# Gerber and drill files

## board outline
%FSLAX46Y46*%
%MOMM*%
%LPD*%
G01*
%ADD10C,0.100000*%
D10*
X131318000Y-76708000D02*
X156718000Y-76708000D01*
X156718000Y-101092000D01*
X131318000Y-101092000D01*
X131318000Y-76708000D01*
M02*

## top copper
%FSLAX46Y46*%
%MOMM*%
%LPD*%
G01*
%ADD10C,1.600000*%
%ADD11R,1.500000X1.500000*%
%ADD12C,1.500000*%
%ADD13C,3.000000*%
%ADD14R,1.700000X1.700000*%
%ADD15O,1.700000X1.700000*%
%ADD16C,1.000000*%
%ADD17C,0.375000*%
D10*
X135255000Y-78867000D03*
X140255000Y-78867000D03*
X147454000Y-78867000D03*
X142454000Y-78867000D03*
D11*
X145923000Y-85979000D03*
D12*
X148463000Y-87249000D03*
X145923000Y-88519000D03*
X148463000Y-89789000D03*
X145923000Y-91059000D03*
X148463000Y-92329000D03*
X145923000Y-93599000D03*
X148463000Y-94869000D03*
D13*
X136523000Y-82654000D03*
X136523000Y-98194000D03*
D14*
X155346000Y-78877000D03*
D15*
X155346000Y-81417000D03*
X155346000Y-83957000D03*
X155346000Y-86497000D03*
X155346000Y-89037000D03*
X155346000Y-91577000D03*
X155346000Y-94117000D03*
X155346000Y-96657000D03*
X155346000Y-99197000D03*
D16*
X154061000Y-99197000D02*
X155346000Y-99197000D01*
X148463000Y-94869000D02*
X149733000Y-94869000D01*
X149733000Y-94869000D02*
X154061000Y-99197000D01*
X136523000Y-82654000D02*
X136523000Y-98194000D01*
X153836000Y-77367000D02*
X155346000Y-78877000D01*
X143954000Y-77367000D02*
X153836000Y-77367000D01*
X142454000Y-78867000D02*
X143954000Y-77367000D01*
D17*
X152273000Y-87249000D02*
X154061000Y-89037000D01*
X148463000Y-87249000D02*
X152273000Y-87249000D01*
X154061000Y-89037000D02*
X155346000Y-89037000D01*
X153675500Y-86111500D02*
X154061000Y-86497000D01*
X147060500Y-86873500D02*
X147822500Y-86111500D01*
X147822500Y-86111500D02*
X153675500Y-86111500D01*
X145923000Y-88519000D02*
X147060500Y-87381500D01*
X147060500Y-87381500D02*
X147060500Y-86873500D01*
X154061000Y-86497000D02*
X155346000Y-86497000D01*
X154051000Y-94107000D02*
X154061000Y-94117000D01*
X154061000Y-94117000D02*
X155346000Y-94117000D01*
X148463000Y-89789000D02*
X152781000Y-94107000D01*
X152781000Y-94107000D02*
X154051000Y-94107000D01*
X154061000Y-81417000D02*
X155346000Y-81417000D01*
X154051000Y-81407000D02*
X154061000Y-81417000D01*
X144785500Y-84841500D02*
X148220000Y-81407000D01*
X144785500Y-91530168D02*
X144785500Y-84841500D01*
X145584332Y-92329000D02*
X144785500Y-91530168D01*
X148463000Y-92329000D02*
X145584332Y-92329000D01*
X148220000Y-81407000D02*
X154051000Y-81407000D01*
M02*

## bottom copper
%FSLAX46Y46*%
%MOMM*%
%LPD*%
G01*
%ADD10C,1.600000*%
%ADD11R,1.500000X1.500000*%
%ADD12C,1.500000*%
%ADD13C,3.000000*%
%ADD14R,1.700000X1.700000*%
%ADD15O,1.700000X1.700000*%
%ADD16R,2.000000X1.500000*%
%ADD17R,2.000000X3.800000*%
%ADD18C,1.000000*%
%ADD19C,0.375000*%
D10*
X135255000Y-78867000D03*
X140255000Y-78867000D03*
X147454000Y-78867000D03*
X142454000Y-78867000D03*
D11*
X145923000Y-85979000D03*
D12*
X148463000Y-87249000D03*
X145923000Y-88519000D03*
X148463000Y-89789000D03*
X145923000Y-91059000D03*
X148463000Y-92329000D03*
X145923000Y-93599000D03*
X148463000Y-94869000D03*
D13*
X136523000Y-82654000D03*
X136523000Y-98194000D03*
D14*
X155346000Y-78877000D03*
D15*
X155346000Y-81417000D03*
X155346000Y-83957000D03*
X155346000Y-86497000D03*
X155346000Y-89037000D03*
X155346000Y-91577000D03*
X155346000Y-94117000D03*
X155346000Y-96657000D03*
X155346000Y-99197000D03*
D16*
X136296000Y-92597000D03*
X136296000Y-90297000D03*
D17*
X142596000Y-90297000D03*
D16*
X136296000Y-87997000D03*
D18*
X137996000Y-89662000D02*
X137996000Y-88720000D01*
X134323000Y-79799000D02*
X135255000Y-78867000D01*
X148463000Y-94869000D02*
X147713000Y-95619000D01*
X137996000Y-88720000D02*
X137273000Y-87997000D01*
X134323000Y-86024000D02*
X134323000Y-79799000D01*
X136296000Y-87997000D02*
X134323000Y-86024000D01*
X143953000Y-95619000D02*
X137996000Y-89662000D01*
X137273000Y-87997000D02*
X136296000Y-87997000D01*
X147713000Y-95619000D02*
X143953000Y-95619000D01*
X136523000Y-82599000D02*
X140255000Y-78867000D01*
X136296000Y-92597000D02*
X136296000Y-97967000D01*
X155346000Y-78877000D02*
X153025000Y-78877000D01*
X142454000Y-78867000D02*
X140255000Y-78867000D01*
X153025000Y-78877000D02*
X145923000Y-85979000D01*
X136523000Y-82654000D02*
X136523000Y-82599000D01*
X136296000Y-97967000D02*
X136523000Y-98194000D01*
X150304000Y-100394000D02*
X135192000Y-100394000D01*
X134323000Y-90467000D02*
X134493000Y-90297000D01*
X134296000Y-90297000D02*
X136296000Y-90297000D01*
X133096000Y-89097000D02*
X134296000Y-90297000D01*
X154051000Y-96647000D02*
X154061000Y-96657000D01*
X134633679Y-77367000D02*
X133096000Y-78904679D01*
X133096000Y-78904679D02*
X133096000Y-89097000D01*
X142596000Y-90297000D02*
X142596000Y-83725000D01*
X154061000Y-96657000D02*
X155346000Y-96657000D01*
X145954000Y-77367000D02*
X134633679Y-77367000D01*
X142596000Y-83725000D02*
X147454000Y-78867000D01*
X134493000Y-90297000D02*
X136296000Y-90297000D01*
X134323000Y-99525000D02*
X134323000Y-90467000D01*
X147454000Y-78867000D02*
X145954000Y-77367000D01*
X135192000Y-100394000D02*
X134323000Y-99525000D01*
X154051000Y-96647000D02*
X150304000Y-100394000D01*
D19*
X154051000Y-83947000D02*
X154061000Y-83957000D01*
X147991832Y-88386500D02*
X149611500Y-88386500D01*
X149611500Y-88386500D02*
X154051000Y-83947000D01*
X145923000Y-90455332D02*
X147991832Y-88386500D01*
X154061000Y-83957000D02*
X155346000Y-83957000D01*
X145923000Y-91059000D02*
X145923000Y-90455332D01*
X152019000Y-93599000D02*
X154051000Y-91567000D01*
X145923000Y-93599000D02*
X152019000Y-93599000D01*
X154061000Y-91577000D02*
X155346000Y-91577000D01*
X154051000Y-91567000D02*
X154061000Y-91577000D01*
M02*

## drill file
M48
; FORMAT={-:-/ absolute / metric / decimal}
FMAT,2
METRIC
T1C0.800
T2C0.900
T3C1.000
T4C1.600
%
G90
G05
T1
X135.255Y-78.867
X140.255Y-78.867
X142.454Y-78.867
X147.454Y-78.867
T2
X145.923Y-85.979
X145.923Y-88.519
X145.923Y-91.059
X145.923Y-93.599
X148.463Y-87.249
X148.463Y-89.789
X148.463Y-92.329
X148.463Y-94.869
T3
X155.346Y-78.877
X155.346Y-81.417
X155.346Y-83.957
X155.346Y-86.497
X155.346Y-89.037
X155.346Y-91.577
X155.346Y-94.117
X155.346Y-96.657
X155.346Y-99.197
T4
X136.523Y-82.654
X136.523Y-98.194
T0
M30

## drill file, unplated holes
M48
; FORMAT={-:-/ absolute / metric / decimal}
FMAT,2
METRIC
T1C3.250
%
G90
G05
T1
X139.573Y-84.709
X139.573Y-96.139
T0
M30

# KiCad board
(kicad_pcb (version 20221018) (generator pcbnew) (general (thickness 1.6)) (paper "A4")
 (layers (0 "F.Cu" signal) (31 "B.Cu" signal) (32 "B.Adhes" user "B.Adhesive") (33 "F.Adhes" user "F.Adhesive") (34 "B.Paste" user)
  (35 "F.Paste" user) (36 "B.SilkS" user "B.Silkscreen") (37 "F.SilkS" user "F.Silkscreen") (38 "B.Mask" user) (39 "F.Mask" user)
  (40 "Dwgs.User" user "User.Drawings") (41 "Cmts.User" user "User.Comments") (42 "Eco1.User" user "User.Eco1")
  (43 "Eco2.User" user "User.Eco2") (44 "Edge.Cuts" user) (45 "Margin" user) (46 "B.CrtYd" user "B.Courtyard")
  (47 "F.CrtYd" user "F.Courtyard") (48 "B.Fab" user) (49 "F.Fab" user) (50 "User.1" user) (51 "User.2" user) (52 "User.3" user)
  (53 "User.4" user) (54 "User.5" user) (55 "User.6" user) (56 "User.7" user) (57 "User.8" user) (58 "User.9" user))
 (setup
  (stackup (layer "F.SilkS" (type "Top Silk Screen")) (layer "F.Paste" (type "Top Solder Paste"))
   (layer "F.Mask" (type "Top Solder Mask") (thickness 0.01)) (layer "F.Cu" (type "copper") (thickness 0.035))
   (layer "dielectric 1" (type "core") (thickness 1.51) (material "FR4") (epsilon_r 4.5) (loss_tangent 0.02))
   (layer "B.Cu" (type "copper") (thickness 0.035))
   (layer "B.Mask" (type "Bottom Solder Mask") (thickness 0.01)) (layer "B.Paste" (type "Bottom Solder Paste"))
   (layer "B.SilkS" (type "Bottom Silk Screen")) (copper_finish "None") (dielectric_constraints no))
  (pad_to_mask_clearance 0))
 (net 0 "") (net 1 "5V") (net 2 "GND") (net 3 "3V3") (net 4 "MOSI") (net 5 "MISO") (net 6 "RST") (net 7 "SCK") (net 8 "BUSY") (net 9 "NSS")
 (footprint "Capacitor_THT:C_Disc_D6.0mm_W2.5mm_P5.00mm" (layer "F.Cu") (at 135.255 78.867)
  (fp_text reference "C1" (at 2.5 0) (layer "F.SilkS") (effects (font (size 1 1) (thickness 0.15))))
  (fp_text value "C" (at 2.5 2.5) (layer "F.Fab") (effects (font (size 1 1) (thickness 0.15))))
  (pad "1" thru_hole circle (at 0 0) (size 1.6 1.6) (drill 0.8) (layers "*.Cu" "*.Mask") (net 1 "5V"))
  (pad "2" thru_hole circle (at 5 0) (size 1.6 1.6) (drill 0.8) (layers "*.Cu" "*.Mask") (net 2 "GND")))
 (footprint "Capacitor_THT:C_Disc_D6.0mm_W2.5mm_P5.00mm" (layer "F.Cu") (at 147.454 78.867 180)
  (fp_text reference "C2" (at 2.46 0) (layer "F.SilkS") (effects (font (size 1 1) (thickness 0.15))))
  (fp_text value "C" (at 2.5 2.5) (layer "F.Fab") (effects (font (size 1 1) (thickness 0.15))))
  (pad "1" thru_hole circle (at 0 0 180) (size 1.6 1.6) (drill 0.8) (layers "*.Cu" "*.Mask") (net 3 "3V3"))
  (pad "2" thru_hole circle (at 5 0 180) (size 1.6 1.6) (drill 0.8) (layers "*.Cu" "*.Mask") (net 2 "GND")))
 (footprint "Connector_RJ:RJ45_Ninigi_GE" (layer "F.Cu") (at 145.923 85.979 -90)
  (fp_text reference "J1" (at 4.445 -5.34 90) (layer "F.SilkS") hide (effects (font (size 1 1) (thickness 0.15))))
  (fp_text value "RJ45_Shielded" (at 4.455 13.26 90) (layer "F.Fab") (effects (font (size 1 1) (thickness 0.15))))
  (pad "" np_thru_hole circle (at -1.27 6.35 270) (size 3.25 3.25) (drill 3.25) (layers "*.Cu" "*.Mask"))
  (pad "" np_thru_hole circle (at 10.16 6.35 90) (size 3.25 3.25) (drill 3.25) (layers "*.Cu" "*.Mask"))
  (pad "1" thru_hole rect (at 0 0 90) (size 1.5 1.5) (drill 0.9) (layers "*.Cu" "*.Mask") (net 2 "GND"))
  (pad "2" thru_hole circle (at 1.27 -2.54 90) (size 1.5 1.5) (drill 0.9) (layers "*.Cu" "*.Mask") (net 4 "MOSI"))
  (pad "3" thru_hole circle (at 2.54 0 90) (size 1.5 1.5) (drill 0.9) (layers "*.Cu" "*.Mask") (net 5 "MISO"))
  (pad "4" thru_hole circle (at 3.81 -2.54 90) (size 1.5 1.5) (drill 0.9) (layers "*.Cu" "*.Mask") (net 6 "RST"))
  (pad "5" thru_hole circle (at 5.08 0 90) (size 1.5 1.5) (drill 0.9) (layers "*.Cu" "*.Mask") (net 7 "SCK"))
  (pad "6" thru_hole circle (at 6.35 -2.54 90) (size 1.5 1.5) (drill 0.9) (layers "*.Cu" "*.Mask") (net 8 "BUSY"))
  (pad "7" thru_hole circle (at 7.62 0 90) (size 1.5 1.5) (drill 0.9) (layers "*.Cu" "*.Mask") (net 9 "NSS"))
  (pad "8" thru_hole circle (at 8.89 -2.54 90) (size 1.5 1.5) (drill 0.9) (layers "*.Cu" "*.Mask") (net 1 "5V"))
  (pad "SH" thru_hole circle (at -3.325 9.4 270) (size 3 3) (drill 1.6) (layers "*.Cu" "*.Mask") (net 2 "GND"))
  (pad "SH" thru_hole circle (at 12.215 9.4 90) (size 3 3) (drill 1.6) (layers "*.Cu" "*.Mask") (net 2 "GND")))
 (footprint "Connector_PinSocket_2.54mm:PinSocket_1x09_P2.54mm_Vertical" (layer "F.Cu") (at 155.346 78.877)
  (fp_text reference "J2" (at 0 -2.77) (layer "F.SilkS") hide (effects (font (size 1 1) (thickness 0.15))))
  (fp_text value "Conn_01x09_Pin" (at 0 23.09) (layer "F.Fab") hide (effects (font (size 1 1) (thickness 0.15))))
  (pad "1" thru_hole rect (at 0 0) (size 1.7 1.7) (drill 1) (layers "*.Cu" "*.Mask") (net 2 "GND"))
  (pad "2" thru_hole oval (at 0 2.54) (size 1.7 1.7) (drill 1) (layers "*.Cu" "*.Mask") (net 8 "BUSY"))
  (pad "3" thru_hole oval (at 0 5.08) (size 1.7 1.7) (drill 1) (layers "*.Cu" "*.Mask") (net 7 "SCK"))
  (pad "4" thru_hole oval (at 0 7.62) (size 1.7 1.7) (drill 1) (layers "*.Cu" "*.Mask") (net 5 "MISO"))
  (pad "5" thru_hole oval (at 0 10.16) (size 1.7 1.7) (drill 1) (layers "*.Cu" "*.Mask") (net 4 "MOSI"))
  (pad "6" thru_hole oval (at 0 12.7) (size 1.7 1.7) (drill 1) (layers "*.Cu" "*.Mask") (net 9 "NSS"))
  (pad "7" thru_hole oval (at 0 15.24) (size 1.7 1.7) (drill 1) (layers "*.Cu" "*.Mask") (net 6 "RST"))
  (pad "8" thru_hole oval (at 0 17.78) (size 1.7 1.7) (drill 1) (layers "*.Cu" "*.Mask") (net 3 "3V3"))
  (pad "9" thru_hole oval (at 0 20.32) (size 1.7 1.7) (drill 1) (layers "*.Cu" "*.Mask") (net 1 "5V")))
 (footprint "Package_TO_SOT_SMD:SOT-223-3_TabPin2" (layer "B.Cu") (at 139.446 90.297)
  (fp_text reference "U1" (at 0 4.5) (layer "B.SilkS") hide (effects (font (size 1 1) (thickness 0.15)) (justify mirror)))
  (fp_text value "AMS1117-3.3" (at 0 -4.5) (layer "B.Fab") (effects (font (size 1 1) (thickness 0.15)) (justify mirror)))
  (pad "1" smd rect (at -3.15 2.3) (size 2 1.5) (layers "B.Cu" "B.Paste" "B.Mask") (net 2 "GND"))
  (pad "2" smd rect (at -3.15 0) (size 2 1.5) (layers "B.Cu" "B.Paste" "B.Mask") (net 3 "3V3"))
  (pad "2" smd rect (at 3.15 0) (size 2 3.8) (layers "B.Cu" "B.Paste" "B.Mask") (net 3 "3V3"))
  (pad "3" smd rect (at -3.15 -2.3) (size 2 1.5) (layers "B.Cu" "B.Paste" "B.Mask") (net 1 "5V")))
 (gr_rect (start 131.318 76.708) (end 156.718 101.092) (stroke (width 0.1) (type default)) (fill none) (layer "Edge.Cuts"))
 (segment (start 154.061 99.197) (end 155.346 99.197) (width 1) (layer "F.Cu") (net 1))
 (segment (start 148.463 94.869) (end 149.733 94.869) (width 1) (layer "F.Cu") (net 1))
 (segment (start 149.733 94.869) (end 154.061 99.197) (width 1) (layer "F.Cu") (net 1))
 (segment (start 137.996 89.662) (end 137.996 88.72) (width 1) (layer "B.Cu") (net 1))
 (segment (start 134.323 79.799) (end 135.255 78.867) (width 1) (layer "B.Cu") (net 1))
 (segment (start 148.463 94.869) (end 147.713 95.619) (width 1) (layer "B.Cu") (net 1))
 (segment (start 137.996 88.72) (end 137.273 87.997) (width 1) (layer "B.Cu") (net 1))
 (segment (start 134.323 86.024) (end 134.323 79.799) (width 1) (layer "B.Cu") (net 1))
 (segment (start 136.296 87.997) (end 134.323 86.024) (width 1) (layer "B.Cu") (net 1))
 (segment (start 143.953 95.619) (end 137.996 89.662) (width 1) (layer "B.Cu") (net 1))
 (segment (start 137.273 87.997) (end 136.296 87.997) (width 1) (layer "B.Cu") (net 1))
 (segment (start 147.713 95.619) (end 143.953 95.619) (width 1) (layer "B.Cu") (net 1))
 (segment (start 136.523 82.654) (end 136.523 98.194) (width 1) (layer "F.Cu") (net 2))
 (segment (start 153.836 77.367) (end 155.346 78.877) (width 1) (layer "F.Cu") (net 2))
 (segment (start 143.954 77.367) (end 153.836 77.367) (width 1) (layer "F.Cu") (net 2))
 (segment (start 142.454 78.867) (end 143.954 77.367) (width 1) (layer "F.Cu") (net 2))
 (segment (start 136.523 82.599) (end 140.255 78.867) (width 1) (layer "B.Cu") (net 2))
 (segment (start 136.296 92.597) (end 136.296 97.967) (width 1) (layer "B.Cu") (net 2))
 (segment (start 155.346 78.877) (end 153.025 78.877) (width 1) (layer "B.Cu") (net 2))
 (segment (start 142.454 78.867) (end 140.255 78.867) (width 1) (layer "B.Cu") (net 2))
 (segment (start 153.025 78.877) (end 145.923 85.979) (width 1) (layer "B.Cu") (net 2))
 (segment (start 136.523 82.654) (end 136.523 82.599) (width 1) (layer "B.Cu") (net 2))
 (segment (start 136.296 97.967) (end 136.523 98.194) (width 1) (layer "B.Cu") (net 2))
 (segment (start 150.304 100.394) (end 135.192 100.394) (width 1) (layer "B.Cu") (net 3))
 (segment (start 134.323 90.467) (end 134.493 90.297) (width 1) (layer "B.Cu") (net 3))
 (segment (start 134.296 90.297) (end 136.296 90.297) (width 1) (layer "B.Cu") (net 3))
 (segment (start 133.096 89.097) (end 134.296 90.297) (width 1) (layer "B.Cu") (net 3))
 (segment (start 154.051 96.647) (end 154.061 96.657) (width 1) (layer "B.Cu") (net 3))
 (segment (start 134.633679 77.367) (end 133.096 78.904679) (width 1) (layer "B.Cu") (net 3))
 (segment (start 133.096 78.904679) (end 133.096 89.097) (width 1) (layer "B.Cu") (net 3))
 (segment (start 142.596 90.297) (end 142.596 83.725) (width 1) (layer "B.Cu") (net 3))
 (segment (start 154.061 96.657) (end 155.346 96.657) (width 1) (layer "B.Cu") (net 3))
 (segment (start 145.954 77.367) (end 134.633679 77.367) (width 1) (layer "B.Cu") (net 3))
 (segment (start 142.596 83.725) (end 147.454 78.867) (width 1) (layer "B.Cu") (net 3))
 (segment (start 134.493 90.297) (end 136.296 90.297) (width 1) (layer "B.Cu") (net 3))
 (segment (start 134.323 99.525) (end 134.323 90.467) (width 1) (layer "B.Cu") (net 3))
 (segment (start 147.454 78.867) (end 145.954 77.367) (width 1) (layer "B.Cu") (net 3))
 (segment (start 135.192 100.394) (end 134.323 99.525) (width 1) (layer "B.Cu") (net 3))
 (segment (start 154.051 96.647) (end 150.304 100.394) (width 1) (layer "B.Cu") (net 3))
 (segment (start 152.273 87.249) (end 154.061 89.037) (width 0.375) (layer "F.Cu") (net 4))
 (segment (start 148.463 87.249) (end 152.273 87.249) (width 0.375) (layer "F.Cu") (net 4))
 (segment (start 154.061 89.037) (end 155.346 89.037) (width 0.375) (layer "F.Cu") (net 4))
 (segment (start 153.6755 86.1115) (end 154.061 86.497) (width 0.375) (layer "F.Cu") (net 5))
 (segment (start 147.0605 86.8735) (end 147.8225 86.1115) (width 0.375) (layer "F.Cu") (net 5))
 (segment (start 147.8225 86.1115) (end 153.6755 86.1115) (width 0.375) (layer "F.Cu") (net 5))
 (segment (start 145.923 88.519) (end 147.0605 87.3815) (width 0.375) (layer "F.Cu") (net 5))
 (segment (start 147.0605 87.3815) (end 147.0605 86.8735) (width 0.375) (layer "F.Cu") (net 5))
 (segment (start 154.061 86.497) (end 155.346 86.497) (width 0.375) (layer "F.Cu") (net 5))
 (segment (start 154.051 94.107) (end 154.061 94.117) (width 0.375) (layer "F.Cu") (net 6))
 (segment (start 154.061 94.117) (end 155.346 94.117) (width 0.375) (layer "F.Cu") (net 6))
 (segment (start 148.463 89.789) (end 152.781 94.107) (width 0.375) (layer "F.Cu") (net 6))
 (segment (start 152.781 94.107) (end 154.051 94.107) (width 0.375) (layer "F.Cu") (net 6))
 (segment (start 154.051 83.947) (end 154.061 83.957) (width 0.375) (layer "B.Cu") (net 7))
 (segment (start 147.991832 88.3865) (end 149.6115 88.3865) (width 0.375) (layer "B.Cu") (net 7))
 (segment (start 149.6115 88.3865) (end 154.051 83.947) (width 0.375) (layer "B.Cu") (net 7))
 (segment (start 145.923 90.455332) (end 147.991832 88.3865) (width 0.375) (layer "B.Cu") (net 7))
 (segment (start 154.061 83.957) (end 155.346 83.957) (width 0.375) (layer "B.Cu") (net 7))
 (segment (start 145.923 91.059) (end 145.923 90.455332) (width 0.375) (layer "B.Cu") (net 7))
 (segment (start 154.061 81.417) (end 155.346 81.417) (width 0.375) (layer "F.Cu") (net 8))
 (segment (start 154.051 81.407) (end 154.061 81.417) (width 0.375) (layer "F.Cu") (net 8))
 (segment (start 144.7855 84.8415) (end 148.22 81.407) (width 0.375) (layer "F.Cu") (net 8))
 (segment (start 144.7855 91.530168) (end 144.7855 84.8415) (width 0.375) (layer "F.Cu") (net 8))
 (segment (start 145.584332 92.329) (end 144.7855 91.530168) (width 0.375) (layer "F.Cu") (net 8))
 (segment (start 148.463 92.329) (end 145.584332 92.329) (width 0.375) (layer "F.Cu") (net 8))
 (segment (start 148.22 81.407) (end 154.051 81.407) (width 0.375) (layer "F.Cu") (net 8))
 (segment (start 152.019 93.599) (end 154.051 91.567) (width 0.375) (layer "B.Cu") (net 9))
 (segment (start 145.923 93.599) (end 152.019 93.599) (width 0.375) (layer "B.Cu") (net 9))
 (segment (start 154.061 91.577) (end 155.346 91.577) (width 0.375) (layer "B.Cu") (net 9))
 (segment (start 154.051 91.567) (end 154.061 91.577) (width 0.375) (layer "B.Cu") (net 9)))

